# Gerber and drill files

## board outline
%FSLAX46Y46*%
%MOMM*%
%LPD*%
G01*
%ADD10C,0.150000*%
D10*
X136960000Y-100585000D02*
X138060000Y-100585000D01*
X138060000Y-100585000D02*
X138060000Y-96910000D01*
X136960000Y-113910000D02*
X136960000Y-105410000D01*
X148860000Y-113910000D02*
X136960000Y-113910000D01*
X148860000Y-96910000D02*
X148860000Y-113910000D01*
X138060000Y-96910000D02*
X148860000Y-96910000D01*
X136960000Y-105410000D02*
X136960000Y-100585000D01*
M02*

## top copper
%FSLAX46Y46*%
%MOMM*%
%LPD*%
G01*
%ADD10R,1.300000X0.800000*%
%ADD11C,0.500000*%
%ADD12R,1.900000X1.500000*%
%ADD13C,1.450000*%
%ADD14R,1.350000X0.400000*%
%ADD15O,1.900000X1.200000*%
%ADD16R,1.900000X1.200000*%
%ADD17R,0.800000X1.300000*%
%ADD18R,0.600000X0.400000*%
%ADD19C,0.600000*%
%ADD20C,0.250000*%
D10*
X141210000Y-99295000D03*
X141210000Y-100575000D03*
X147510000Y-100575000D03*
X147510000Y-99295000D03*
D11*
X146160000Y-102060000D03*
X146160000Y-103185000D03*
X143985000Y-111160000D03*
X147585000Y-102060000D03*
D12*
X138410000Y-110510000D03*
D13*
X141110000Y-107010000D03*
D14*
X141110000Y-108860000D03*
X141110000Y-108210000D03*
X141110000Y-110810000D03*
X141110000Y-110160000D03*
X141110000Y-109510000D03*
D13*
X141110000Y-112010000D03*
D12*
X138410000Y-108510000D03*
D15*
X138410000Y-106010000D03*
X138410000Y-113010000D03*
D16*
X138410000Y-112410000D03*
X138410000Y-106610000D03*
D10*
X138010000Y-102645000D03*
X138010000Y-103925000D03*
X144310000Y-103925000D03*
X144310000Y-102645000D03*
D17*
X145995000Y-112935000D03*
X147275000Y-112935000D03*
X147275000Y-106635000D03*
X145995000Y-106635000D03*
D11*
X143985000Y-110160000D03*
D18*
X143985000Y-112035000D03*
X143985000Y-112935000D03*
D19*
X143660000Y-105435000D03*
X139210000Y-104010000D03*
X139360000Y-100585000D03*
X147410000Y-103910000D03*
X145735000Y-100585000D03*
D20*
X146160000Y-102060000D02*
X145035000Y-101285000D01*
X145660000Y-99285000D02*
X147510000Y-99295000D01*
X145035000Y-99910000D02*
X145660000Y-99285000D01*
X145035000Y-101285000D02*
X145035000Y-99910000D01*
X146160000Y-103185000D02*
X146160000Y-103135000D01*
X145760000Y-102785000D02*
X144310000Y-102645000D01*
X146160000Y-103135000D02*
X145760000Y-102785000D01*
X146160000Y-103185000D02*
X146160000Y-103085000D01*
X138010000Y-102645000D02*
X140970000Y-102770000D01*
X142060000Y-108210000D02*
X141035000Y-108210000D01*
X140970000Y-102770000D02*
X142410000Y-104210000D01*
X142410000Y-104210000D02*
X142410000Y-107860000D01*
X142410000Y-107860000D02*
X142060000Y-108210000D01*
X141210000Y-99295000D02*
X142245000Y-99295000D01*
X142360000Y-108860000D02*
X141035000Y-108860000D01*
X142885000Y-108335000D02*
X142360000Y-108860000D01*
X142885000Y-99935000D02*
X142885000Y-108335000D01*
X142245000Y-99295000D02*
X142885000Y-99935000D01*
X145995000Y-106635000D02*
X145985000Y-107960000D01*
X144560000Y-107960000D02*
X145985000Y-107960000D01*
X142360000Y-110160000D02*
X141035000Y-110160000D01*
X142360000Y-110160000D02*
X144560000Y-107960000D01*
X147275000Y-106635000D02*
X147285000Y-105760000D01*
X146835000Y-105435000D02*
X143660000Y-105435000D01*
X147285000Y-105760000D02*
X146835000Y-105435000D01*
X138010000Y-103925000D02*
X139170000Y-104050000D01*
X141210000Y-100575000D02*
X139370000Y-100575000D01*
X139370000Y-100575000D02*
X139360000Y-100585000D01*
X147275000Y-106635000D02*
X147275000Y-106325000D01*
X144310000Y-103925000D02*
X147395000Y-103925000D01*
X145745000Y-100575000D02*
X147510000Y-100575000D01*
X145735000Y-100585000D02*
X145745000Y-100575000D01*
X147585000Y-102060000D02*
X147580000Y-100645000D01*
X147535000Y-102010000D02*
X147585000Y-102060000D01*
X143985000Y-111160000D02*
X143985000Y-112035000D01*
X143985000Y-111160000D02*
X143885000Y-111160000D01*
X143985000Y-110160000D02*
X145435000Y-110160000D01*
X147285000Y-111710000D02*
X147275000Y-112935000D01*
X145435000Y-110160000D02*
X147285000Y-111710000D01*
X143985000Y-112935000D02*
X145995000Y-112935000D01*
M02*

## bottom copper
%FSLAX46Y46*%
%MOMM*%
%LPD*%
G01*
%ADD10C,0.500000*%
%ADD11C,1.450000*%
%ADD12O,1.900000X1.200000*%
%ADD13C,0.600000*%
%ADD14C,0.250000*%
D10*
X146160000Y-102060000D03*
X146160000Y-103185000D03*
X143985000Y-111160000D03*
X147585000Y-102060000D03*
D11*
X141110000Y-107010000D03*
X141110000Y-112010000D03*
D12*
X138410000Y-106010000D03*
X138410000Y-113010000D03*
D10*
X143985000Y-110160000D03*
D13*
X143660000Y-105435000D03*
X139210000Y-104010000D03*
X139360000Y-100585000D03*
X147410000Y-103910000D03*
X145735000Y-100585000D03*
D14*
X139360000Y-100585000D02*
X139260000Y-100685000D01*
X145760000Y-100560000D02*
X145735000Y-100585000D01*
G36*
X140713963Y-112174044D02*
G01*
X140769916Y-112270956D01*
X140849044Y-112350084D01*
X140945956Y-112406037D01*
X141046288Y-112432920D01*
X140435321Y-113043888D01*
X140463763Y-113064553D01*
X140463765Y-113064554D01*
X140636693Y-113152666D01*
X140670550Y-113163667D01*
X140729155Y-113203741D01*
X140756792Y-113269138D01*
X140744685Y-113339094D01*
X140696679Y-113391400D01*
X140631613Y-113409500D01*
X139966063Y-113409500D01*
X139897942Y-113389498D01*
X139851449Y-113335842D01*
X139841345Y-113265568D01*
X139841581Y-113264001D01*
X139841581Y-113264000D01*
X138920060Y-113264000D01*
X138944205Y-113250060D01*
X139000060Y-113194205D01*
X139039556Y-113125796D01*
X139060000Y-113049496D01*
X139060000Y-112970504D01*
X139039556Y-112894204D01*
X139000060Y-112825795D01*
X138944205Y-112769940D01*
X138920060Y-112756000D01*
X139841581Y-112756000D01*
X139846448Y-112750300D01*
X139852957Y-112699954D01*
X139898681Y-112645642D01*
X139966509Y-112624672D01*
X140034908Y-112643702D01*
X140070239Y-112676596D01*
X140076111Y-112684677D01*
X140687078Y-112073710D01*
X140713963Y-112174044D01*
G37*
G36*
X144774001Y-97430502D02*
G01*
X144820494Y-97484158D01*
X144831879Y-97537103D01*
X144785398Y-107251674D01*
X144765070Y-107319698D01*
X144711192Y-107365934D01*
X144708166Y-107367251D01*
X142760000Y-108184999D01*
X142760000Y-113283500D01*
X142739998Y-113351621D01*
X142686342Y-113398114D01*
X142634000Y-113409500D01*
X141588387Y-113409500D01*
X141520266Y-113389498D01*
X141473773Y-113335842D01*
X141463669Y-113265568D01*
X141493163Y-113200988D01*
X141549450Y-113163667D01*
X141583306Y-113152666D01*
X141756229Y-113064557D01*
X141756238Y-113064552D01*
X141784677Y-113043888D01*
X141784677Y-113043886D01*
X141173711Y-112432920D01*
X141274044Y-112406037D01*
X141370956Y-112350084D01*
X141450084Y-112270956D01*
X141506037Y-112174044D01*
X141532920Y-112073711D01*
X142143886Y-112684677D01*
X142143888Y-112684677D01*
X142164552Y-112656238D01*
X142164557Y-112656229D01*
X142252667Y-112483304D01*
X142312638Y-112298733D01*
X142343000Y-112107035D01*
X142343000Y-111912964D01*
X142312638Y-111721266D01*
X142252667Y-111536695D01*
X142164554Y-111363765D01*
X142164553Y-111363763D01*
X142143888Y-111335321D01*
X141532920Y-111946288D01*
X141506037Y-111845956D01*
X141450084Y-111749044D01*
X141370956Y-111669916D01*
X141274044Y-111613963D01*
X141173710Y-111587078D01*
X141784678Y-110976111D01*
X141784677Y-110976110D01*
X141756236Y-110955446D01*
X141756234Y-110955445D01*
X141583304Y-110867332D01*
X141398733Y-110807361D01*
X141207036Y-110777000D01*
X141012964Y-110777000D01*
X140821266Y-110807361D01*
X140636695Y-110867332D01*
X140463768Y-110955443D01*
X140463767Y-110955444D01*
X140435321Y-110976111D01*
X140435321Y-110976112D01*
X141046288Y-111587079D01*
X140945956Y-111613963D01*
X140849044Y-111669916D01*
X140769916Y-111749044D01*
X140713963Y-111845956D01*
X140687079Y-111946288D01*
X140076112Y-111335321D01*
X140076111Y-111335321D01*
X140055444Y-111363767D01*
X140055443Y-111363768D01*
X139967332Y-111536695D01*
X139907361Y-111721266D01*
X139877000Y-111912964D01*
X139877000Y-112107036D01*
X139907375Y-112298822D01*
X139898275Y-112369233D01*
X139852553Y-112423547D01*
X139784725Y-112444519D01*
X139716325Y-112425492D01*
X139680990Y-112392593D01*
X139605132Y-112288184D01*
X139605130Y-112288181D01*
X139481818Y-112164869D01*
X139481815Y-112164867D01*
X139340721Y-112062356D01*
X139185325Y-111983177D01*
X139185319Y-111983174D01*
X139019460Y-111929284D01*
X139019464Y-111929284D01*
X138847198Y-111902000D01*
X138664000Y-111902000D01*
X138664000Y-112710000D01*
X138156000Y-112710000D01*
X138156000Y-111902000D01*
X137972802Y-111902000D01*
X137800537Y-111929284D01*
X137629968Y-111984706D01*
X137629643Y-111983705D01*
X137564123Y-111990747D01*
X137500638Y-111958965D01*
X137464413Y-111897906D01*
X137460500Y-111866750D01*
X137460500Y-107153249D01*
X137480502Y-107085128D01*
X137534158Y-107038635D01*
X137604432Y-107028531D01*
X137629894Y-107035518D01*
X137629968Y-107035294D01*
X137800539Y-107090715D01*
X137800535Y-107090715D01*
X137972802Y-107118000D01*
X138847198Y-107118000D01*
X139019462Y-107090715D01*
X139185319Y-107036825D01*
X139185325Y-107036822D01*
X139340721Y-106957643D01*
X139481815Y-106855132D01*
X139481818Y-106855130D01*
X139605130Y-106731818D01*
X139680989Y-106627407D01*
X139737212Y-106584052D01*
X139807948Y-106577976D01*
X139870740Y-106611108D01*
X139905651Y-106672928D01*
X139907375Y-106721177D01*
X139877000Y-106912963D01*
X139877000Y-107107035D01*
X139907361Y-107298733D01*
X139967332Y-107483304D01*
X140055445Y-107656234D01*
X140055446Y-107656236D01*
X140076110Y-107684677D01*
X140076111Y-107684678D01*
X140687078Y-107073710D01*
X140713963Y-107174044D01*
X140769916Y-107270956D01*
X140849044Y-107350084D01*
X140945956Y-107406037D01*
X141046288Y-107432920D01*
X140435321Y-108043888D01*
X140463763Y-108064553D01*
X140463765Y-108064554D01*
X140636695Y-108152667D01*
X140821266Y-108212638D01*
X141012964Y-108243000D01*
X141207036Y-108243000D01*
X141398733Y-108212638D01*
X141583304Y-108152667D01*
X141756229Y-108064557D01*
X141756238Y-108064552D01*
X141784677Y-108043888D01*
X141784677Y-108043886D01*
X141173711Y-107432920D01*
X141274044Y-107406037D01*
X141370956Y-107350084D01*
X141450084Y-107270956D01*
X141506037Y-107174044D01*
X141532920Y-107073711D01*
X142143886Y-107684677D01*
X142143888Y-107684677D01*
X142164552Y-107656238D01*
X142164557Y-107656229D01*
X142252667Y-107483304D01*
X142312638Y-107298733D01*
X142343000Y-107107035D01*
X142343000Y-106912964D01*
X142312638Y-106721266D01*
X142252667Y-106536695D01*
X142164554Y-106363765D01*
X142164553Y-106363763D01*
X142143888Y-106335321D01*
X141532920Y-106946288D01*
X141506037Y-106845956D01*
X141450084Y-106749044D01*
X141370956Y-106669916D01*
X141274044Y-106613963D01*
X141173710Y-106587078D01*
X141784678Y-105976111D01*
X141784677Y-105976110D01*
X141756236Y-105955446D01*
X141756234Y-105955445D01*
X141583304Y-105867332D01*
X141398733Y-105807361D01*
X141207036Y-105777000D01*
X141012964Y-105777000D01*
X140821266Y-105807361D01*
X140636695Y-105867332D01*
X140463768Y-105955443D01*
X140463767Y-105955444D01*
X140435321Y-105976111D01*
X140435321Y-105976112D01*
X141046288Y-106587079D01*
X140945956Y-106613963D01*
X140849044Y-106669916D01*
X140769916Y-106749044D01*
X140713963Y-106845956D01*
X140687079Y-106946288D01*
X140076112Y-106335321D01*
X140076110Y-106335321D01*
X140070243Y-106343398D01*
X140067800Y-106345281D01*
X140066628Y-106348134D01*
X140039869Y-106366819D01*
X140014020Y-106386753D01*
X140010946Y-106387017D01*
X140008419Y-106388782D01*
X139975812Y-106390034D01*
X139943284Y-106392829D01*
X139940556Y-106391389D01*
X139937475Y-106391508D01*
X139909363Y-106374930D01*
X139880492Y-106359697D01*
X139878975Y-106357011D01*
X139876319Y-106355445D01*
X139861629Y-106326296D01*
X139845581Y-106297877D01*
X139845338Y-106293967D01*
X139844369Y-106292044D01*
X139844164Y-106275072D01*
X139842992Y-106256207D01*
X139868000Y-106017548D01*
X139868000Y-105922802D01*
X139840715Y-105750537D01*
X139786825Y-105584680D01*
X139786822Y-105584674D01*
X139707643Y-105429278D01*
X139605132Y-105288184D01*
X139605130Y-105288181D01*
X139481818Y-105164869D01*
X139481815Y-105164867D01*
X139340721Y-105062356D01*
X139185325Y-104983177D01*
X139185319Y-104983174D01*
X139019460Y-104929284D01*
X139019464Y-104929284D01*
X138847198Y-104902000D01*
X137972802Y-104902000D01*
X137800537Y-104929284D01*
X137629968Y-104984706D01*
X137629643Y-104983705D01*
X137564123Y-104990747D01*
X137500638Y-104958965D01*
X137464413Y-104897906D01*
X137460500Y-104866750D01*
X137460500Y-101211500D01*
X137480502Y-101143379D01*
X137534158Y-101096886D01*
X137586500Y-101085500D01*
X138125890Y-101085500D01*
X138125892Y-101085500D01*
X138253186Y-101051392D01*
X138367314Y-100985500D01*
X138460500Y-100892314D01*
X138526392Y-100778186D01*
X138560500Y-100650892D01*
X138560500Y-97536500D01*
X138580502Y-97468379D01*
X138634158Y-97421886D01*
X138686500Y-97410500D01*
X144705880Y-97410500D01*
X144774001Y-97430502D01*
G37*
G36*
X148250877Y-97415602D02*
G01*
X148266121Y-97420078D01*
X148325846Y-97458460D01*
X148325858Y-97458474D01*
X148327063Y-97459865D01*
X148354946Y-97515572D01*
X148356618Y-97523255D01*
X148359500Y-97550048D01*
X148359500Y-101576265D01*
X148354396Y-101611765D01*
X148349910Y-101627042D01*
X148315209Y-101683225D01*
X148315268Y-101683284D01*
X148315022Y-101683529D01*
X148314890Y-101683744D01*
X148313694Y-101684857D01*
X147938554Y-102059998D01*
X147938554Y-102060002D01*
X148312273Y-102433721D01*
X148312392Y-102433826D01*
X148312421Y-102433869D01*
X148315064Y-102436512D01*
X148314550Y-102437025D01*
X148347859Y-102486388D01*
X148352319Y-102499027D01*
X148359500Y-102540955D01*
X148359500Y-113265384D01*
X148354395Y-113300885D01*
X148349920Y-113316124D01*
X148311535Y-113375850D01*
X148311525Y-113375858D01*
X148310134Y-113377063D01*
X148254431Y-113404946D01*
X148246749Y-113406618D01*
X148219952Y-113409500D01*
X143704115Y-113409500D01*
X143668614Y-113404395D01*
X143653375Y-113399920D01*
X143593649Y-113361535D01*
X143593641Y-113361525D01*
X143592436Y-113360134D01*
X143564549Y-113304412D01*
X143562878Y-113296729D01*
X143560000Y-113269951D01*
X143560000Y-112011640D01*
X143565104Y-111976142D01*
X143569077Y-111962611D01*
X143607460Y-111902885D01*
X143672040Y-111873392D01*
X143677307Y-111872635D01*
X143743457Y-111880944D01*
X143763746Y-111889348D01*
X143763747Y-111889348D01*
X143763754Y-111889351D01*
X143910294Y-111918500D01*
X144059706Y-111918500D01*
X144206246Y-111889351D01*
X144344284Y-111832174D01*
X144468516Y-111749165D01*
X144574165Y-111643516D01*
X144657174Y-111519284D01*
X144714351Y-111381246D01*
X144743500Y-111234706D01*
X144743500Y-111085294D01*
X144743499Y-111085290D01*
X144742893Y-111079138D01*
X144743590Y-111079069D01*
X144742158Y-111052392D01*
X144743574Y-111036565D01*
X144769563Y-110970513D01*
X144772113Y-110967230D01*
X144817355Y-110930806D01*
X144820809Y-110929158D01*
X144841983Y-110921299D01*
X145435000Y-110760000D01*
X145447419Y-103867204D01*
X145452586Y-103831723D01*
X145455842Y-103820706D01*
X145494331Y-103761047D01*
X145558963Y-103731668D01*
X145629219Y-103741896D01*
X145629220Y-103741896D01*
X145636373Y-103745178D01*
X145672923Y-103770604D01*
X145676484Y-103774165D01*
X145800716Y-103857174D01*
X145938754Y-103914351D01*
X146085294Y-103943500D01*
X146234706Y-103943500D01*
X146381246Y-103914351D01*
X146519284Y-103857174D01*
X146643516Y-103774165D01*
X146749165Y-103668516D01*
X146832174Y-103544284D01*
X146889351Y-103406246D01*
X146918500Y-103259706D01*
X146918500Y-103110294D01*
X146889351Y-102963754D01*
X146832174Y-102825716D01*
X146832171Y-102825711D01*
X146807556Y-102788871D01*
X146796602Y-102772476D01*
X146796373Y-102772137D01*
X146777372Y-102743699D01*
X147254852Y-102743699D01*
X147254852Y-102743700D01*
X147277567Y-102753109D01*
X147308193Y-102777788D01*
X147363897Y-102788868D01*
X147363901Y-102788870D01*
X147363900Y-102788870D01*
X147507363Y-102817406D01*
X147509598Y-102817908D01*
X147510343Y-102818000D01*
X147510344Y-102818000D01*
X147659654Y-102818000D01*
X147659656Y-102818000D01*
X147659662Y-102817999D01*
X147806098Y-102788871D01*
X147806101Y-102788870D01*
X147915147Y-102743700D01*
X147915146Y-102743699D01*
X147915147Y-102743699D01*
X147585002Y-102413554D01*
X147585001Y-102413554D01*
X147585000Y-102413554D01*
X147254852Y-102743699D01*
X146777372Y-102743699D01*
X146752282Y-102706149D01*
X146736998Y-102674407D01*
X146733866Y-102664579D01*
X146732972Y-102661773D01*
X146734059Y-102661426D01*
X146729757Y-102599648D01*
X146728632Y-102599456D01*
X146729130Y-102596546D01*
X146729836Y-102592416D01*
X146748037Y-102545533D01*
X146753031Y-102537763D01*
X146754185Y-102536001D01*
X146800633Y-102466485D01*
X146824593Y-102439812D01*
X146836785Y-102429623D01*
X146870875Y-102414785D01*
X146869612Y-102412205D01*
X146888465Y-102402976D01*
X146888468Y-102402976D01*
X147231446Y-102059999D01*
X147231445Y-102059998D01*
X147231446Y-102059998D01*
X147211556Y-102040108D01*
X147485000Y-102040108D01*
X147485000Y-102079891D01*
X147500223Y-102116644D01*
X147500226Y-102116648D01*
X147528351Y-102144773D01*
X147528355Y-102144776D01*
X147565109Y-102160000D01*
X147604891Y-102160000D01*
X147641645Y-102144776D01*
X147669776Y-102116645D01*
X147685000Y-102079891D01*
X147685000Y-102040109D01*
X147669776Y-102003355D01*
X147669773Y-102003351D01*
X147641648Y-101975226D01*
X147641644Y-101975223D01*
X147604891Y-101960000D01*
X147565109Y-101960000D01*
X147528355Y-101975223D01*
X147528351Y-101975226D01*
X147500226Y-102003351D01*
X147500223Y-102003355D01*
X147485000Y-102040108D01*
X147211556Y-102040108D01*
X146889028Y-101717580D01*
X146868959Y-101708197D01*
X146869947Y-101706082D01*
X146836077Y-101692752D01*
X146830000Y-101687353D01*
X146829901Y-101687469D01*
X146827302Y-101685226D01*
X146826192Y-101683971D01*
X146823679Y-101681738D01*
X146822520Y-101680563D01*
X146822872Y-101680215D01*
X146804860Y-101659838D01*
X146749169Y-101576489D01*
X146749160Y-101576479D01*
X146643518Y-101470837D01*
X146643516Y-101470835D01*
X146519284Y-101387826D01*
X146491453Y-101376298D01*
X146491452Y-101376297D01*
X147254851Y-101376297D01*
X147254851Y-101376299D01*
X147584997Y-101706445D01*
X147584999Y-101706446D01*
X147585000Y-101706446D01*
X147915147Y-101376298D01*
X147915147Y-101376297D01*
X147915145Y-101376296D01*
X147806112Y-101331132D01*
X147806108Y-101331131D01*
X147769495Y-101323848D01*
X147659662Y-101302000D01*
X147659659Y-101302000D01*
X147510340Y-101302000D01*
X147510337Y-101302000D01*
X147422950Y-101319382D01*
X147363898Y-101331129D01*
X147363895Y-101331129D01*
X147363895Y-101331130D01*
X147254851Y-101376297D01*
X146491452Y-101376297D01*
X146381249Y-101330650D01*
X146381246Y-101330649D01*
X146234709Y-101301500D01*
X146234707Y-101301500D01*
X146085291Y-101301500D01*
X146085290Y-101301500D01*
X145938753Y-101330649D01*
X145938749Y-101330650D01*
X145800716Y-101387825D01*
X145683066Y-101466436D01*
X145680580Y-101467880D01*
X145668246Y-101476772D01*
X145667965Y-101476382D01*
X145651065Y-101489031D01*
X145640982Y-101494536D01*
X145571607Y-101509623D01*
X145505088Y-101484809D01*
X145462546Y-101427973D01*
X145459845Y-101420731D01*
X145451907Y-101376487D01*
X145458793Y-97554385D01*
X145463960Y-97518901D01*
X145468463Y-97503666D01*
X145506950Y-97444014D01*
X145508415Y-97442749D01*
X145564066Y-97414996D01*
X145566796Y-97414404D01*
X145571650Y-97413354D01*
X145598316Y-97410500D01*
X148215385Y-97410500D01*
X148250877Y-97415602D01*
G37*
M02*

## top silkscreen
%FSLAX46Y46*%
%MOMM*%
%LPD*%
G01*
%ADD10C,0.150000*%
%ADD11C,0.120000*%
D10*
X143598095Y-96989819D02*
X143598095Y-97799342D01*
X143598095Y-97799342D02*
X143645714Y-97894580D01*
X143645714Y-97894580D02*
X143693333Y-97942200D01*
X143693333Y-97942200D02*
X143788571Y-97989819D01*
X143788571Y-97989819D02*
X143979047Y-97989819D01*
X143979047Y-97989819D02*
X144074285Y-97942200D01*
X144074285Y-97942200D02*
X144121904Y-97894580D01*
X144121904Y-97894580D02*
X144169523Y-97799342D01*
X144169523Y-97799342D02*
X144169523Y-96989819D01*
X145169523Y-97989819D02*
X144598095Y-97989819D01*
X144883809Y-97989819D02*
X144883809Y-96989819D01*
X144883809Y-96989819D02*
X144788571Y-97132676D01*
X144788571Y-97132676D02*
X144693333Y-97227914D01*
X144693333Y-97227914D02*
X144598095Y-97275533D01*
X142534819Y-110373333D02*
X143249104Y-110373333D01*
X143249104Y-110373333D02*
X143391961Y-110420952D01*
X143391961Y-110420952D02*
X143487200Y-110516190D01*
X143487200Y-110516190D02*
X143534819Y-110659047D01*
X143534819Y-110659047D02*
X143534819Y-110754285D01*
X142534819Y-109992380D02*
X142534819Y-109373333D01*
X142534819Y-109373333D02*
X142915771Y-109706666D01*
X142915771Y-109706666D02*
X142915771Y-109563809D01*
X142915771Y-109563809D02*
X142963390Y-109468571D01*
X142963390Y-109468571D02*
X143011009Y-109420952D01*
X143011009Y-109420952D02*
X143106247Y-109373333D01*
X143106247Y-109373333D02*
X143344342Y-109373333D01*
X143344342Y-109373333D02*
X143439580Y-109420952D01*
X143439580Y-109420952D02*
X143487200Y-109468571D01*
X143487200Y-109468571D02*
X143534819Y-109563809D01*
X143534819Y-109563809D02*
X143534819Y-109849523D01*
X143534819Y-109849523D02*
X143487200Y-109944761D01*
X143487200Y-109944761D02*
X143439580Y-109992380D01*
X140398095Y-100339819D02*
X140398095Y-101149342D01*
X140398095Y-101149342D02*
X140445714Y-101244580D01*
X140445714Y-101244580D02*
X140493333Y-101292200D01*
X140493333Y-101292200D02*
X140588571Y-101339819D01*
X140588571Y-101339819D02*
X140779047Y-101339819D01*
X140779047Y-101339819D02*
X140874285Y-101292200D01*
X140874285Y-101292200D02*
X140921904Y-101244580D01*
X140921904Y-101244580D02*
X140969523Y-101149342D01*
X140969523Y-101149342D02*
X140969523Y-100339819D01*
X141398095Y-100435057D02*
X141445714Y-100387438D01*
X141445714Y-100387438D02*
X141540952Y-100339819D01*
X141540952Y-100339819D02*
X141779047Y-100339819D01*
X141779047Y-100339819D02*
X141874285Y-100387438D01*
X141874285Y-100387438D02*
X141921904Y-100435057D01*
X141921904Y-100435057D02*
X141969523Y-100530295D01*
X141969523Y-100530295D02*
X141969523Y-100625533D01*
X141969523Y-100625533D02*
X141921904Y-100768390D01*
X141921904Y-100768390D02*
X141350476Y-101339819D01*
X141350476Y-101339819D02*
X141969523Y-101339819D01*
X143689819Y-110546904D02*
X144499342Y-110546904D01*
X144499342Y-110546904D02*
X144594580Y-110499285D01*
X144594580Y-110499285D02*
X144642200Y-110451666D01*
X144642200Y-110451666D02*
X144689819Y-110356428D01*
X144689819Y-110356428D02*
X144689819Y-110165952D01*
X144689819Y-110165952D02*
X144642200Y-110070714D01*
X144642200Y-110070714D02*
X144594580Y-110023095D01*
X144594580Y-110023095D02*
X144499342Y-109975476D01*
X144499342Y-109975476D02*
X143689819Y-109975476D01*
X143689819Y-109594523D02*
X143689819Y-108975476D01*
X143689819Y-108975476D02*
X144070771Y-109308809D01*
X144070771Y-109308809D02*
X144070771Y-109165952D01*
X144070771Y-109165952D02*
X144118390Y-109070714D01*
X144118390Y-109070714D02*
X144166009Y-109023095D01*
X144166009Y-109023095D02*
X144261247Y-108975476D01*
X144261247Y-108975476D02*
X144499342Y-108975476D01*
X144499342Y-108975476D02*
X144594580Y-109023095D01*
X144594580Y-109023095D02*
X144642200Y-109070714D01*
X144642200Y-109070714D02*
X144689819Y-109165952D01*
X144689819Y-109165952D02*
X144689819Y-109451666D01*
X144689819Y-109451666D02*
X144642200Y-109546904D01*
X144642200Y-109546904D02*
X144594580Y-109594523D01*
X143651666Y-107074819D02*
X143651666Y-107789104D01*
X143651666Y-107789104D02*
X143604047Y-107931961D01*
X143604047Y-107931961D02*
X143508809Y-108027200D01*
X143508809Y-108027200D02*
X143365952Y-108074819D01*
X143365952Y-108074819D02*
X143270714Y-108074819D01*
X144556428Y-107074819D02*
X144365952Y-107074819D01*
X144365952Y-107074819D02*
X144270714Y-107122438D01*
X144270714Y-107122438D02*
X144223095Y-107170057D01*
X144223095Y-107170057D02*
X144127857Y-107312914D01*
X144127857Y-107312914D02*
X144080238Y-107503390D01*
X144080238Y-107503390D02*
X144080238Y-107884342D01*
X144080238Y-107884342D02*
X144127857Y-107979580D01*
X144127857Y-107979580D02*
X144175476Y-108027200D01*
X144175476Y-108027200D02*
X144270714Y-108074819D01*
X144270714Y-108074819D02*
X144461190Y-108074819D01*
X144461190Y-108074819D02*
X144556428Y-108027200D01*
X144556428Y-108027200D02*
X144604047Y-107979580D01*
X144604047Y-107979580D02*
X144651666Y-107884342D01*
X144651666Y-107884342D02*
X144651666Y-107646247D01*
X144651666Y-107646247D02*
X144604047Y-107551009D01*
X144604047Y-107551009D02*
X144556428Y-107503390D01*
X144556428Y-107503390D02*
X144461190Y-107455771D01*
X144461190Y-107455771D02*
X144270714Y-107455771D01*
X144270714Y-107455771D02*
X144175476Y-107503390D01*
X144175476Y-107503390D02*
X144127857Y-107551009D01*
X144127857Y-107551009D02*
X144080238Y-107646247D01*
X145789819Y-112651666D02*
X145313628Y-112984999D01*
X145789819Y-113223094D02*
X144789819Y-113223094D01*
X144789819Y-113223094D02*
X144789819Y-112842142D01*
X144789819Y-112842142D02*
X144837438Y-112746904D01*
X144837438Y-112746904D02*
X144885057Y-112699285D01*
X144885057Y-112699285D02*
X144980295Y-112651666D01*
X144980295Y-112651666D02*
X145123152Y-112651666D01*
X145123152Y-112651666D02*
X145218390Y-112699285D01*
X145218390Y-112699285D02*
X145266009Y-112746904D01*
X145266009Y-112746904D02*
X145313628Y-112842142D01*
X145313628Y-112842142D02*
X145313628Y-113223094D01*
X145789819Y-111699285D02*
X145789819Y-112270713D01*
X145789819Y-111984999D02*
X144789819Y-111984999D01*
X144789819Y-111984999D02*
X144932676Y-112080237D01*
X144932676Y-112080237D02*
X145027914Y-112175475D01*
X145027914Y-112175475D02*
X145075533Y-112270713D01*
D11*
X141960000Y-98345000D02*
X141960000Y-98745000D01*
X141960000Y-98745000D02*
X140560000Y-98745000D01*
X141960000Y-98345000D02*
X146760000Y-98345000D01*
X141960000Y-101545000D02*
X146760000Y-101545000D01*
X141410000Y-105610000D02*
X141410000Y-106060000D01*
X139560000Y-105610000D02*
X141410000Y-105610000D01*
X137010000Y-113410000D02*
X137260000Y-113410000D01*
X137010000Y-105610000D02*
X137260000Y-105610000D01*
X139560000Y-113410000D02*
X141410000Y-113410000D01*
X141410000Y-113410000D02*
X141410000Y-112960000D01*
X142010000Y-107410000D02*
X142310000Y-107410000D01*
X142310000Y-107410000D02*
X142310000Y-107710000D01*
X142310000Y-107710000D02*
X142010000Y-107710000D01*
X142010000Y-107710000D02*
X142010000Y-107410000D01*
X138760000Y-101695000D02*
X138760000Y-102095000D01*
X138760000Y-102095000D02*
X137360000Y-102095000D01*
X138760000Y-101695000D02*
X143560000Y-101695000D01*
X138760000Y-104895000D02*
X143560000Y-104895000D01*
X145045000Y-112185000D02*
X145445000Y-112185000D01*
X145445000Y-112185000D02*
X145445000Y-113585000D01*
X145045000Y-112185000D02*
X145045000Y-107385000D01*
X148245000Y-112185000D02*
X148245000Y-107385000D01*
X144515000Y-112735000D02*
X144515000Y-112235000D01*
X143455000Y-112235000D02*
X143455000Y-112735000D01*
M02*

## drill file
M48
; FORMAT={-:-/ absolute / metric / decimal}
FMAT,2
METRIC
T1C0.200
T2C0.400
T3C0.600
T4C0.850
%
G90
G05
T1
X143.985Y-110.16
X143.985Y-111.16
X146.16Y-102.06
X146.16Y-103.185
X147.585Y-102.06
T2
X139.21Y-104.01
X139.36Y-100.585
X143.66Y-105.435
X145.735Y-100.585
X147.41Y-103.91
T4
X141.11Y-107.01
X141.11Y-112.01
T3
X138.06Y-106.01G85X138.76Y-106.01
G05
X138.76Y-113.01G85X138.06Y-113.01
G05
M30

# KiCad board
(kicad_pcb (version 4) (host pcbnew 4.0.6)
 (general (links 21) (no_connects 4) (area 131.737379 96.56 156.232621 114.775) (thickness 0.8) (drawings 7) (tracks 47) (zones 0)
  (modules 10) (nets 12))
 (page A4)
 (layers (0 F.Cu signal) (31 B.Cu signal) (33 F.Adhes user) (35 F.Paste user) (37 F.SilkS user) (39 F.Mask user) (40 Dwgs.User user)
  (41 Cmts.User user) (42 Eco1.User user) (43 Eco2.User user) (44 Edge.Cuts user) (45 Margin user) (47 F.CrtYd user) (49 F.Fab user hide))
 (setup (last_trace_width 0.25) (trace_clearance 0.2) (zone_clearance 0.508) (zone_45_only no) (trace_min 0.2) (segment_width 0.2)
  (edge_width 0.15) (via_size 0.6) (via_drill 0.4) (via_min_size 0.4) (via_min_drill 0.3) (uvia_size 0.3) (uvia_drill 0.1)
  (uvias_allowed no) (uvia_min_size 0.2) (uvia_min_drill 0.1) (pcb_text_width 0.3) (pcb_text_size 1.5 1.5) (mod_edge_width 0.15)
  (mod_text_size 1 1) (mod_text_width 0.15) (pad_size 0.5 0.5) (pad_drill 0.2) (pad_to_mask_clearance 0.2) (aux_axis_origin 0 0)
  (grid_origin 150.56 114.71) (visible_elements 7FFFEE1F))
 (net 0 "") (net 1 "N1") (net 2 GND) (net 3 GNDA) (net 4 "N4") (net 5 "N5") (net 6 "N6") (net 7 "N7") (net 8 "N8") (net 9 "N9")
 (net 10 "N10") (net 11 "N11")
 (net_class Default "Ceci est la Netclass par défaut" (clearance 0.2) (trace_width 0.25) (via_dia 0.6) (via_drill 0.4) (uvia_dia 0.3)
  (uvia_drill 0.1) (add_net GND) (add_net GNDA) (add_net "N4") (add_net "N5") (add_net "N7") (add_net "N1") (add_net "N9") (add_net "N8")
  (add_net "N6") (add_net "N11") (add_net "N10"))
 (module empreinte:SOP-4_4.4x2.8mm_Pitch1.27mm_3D (layer F.Cu) (at 144.36 99.935)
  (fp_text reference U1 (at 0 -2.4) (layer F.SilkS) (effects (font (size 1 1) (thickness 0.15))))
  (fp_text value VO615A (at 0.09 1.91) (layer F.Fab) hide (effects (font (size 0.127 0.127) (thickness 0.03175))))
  (fp_line (start -2.4 -1.59) (end -2.4 -1.19) (layer F.SilkS) (width 0.12))
  (fp_line (start -2.4 -1.19) (end -3.8 -1.19) (layer F.SilkS) (width 0.12))
  (fp_line (start -2.4 -1.59) (end 2.4 -1.59) (layer F.SilkS) (width 0.12))
  (fp_line (start -2.4 1.61) (end 2.4 1.61) (layer F.SilkS) (width 0.12))
  (pad 1 smd rect (at -3.15 -0.64) (size 1.3 0.8) (layers F.Cu F.Paste F.Mask) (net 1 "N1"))
  (pad 2 smd rect (at -3.15 0.64) (size 1.3 0.8) (layers F.Cu F.Paste F.Mask) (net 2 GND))
  (pad 3 smd rect (at 3.15 0.64) (size 1.3 0.8) (layers F.Cu F.Paste F.Mask) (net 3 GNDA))
  (pad 4 smd rect (at 3.15 -0.64) (size 1.3 0.8) (layers F.Cu F.Paste F.Mask) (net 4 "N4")))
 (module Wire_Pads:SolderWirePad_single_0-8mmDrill (layer F.Cu) (at 146.16 102.06)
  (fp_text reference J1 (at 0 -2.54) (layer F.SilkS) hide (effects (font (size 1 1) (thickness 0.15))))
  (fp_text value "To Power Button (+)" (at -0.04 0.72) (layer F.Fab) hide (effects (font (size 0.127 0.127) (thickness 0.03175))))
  (pad 1 thru_hole circle (at 0 0) (size 0.5 0.5) (drill 0.2) (layers *.Cu *.Mask) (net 4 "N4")))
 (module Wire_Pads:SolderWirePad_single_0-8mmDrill (layer F.Cu) (at 146.16 103.185)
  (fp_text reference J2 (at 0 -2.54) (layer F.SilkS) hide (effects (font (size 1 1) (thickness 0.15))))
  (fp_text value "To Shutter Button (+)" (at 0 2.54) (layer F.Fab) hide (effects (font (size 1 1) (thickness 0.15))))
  (pad 1 thru_hole circle (at 0 0) (size 0.5 0.5) (drill 0.2) (layers *.Cu *.Mask) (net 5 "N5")))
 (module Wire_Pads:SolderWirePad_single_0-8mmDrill (layer F.Cu) (at 143.985 111.16)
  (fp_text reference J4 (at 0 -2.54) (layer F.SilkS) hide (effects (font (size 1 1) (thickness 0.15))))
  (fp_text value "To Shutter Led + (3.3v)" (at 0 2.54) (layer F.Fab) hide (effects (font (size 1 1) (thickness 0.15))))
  (pad 1 thru_hole circle (at 0 0) (size 0.5 0.5) (drill 0.2) (layers *.Cu *.Mask) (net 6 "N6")))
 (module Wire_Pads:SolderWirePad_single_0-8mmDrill (layer F.Cu) (at 147.585 102.06)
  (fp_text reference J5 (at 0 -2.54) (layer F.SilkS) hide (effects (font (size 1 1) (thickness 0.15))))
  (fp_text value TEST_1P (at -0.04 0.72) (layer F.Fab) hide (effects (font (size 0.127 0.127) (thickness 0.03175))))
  (pad 1 thru_hole circle (at 0 0) (size 0.5 0.5) (drill 0.2) (layers *.Cu *.Mask) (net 3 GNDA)))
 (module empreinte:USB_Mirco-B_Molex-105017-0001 (layer F.Cu) (at 141.11 109.51 270)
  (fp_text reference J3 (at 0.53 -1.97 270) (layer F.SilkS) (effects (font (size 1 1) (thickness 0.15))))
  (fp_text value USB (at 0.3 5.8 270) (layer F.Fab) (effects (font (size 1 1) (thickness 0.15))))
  (fp_line (start -3.9 -0.3) (end -3.45 -0.3) (layer F.SilkS) (width 0.12))
  (fp_line (start -3.9 1.55) (end -3.9 -0.3) (layer F.SilkS) (width 0.12))
  (fp_line (start 3.9 4.1) (end 3.9 3.85) (layer F.SilkS) (width 0.12))
  (fp_line (start -3.9 4.1) (end -3.9 3.85) (layer F.SilkS) (width 0.12))
  (fp_line (start 3.9 1.55) (end 3.9 -0.3) (layer F.SilkS) (width 0.12))
  (fp_line (start 3.9 -0.3) (end 3.45 -0.3) (layer F.SilkS) (width 0.12))
  (fp_line (start -2.1 -0.9) (end -2.1 -1.2) (layer F.SilkS) (width 0.12))
  (fp_line (start -2.1 -1.2) (end -1.8 -1.2) (layer F.SilkS) (width 0.12))
  (fp_line (start -1.8 -1.2) (end -1.8 -0.9) (layer F.SilkS) (width 0.12))
  (fp_line (start -1.8 -0.9) (end -2.1 -0.9) (layer F.SilkS) (width 0.12))
  (pad 6 smd rect (at 1 2.7 270) (size 1.5 1.9) (layers F.Cu F.Paste F.Mask) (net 2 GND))
  (pad 6 thru_hole circle (at -2.5 0 270) (size 1.45 1.45) (drill 0.85) (layers *.Cu *.Mask) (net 2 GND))
  (pad 2 smd rect (at -0.65 0 270) (size 0.4 1.35) (layers F.Cu F.Paste F.Mask) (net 1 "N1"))
  (pad 1 smd rect (at -1.3 0 270) (size 0.4 1.35) (layers F.Cu F.Paste F.Mask) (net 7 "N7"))
  (pad 5 smd rect (at 1.3 0 270) (size 0.4 1.35) (layers F.Cu F.Paste F.Mask) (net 2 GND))
  (pad 4 smd rect (at 0.65 0 270) (size 0.4 1.35) (layers F.Cu F.Paste F.Mask) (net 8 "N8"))
  (pad 3 smd rect (at 0 0 270) (size 0.4 1.35) (layers F.Cu F.Paste F.Mask) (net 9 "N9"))
  (pad 6 thru_hole circle (at 2.5 0 270) (size 1.45 1.45) (drill 0.85) (layers *.Cu *.Mask) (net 2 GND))
  (pad 6 smd rect (at -1 2.7 270) (size 1.5 1.9) (layers F.Cu F.Paste F.Mask) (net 2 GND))
  (pad 6 thru_hole oval (at -3.5 2.7 90) (size 1.2 1.9) (drill oval 0.6 1.3) (layers *.Cu *.Mask) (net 2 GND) (zone_connect 0))
  (pad 6 thru_hole oval (at 3.5 2.7 270) (size 1.2 1.9) (drill oval 0.6 1.3) (layers *.Cu *.Mask) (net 2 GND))
  (pad 6 smd rect (at 2.9 2.7 270) (size 1.2 1.9) (layers F.Cu F.Mask) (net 2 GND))
  (pad 6 smd rect (at -2.9 2.7 270) (size 1.2 1.9) (layers F.Cu F.Mask) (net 2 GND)))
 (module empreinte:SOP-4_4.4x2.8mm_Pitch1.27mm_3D (layer F.Cu) (at 141.16 103.285)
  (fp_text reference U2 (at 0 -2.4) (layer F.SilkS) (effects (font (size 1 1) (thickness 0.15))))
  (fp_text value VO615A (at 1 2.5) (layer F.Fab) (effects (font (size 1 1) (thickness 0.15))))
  (fp_line (start -2.4 -1.59) (end -2.4 -1.19) (layer F.SilkS) (width 0.12))
  (fp_line (start -2.4 -1.19) (end -3.8 -1.19) (layer F.SilkS) (width 0.12))
  (fp_line (start -2.4 -1.59) (end 2.4 -1.59) (layer F.SilkS) (width 0.12))
  (fp_line (start -2.4 1.61) (end 2.4 1.61) (layer F.SilkS) (width 0.12))
  (pad 1 smd rect (at -3.15 -0.64) (size 1.3 0.8) (layers F.Cu F.Paste F.Mask) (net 7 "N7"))
  (pad 2 smd rect (at -3.15 0.64) (size 1.3 0.8) (layers F.Cu F.Paste F.Mask) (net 2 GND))
  (pad 3 smd rect (at 3.15 0.64) (size 1.3 0.8) (layers F.Cu F.Paste F.Mask) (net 3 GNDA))
  (pad 4 smd rect (at 3.15 -0.64) (size 1.3 0.8) (layers F.Cu F.Paste F.Mask) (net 5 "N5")))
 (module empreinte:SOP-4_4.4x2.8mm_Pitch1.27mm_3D (layer F.Cu) (at 146.635 109.785 90)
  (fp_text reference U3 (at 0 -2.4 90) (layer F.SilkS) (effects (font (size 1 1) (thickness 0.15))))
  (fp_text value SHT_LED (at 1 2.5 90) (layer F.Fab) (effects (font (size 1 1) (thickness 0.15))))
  (fp_line (start -2.4 -1.59) (end -2.4 -1.19) (layer F.SilkS) (width 0.12))
  (fp_line (start -2.4 -1.19) (end -3.8 -1.19) (layer F.SilkS) (width 0.12))
  (fp_line (start -2.4 -1.59) (end 2.4 -1.59) (layer F.SilkS) (width 0.12))
  (fp_line (start -2.4 1.61) (end 2.4 1.61) (layer F.SilkS) (width 0.12))
  (pad 1 smd rect (at -3.15 -0.64 90) (size 1.3 0.8) (layers F.Cu F.Paste F.Mask) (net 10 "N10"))
  (pad 2 smd rect (at -3.15 0.64 90) (size 1.3 0.8) (layers F.Cu F.Paste F.Mask) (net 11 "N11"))
  (pad 3 smd rect (at 3.15 0.64 90) (size 1.3 0.8) (layers F.Cu F.Paste F.Mask) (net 2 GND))
  (pad 4 smd rect (at 3.15 -0.64 90) (size 1.3 0.8) (layers F.Cu F.Paste F.Mask) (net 8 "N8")))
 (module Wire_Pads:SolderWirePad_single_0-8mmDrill (layer F.Cu) (at 143.985 110.16)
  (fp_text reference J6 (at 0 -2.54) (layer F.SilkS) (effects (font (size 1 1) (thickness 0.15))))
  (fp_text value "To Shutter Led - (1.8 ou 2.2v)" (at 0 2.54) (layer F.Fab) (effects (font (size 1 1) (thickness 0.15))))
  (pad 1 thru_hole circle (at 0 0) (size 0.5 0.5) (drill 0.2) (layers *.Cu *.Mask) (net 11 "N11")))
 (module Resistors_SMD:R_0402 (layer F.Cu) (at 143.985 112.485 270)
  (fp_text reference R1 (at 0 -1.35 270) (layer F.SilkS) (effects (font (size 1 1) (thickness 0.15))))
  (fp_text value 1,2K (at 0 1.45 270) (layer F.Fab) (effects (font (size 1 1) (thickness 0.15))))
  (fp_line (start 0.25 -0.53) (end -0.25 -0.53) (layer F.SilkS) (width 0.12))
  (fp_line (start -0.25 0.53) (end 0.25 0.53) (layer F.SilkS) (width 0.12))
  (pad 1 smd rect (at -0.45 0 270) (size 0.4 0.6) (layers F.Cu F.Paste F.Mask) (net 6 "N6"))
  (pad 2 smd rect (at 0.45 0 270) (size 0.4 0.6) (layers F.Cu F.Paste F.Mask) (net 10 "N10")))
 (gr_line (start 136.96 100.585) (end 138.06 100.585) (layer Edge.Cuts) (width 0.15))
 (gr_line (start 138.06 100.585) (end 138.06 96.91) (angle 90) (layer Edge.Cuts) (width 0.15))
 (gr_line (start 136.96 113.91) (end 136.96 105.41) (angle 90) (layer Edge.Cuts) (width 0.15))
 (gr_line (start 148.86 113.91) (end 136.96 113.91) (angle 90) (layer Edge.Cuts) (width 0.15))
 (gr_line (start 148.86 96.91) (end 148.86 113.91) (angle 90) (layer Edge.Cuts) (width 0.15))
 (gr_line (start 138.06 96.91) (end 148.86 96.91) (angle 90) (layer Edge.Cuts) (width 0.15))
 (gr_line (start 136.96 105.41) (end 136.96 100.585) (angle 90) (layer Edge.Cuts) (width 0.15))
 (segment (start 146.16 102.06) (end 145.035 101.285) (width 0.25) (layer F.Cu) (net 4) (status 10))
 (segment (start 145.66 99.285) (end 147.51 99.295) (width 0.25) (layer F.Cu) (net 4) (status 20))
 (segment (start 145.035 99.91) (end 145.66 99.285) (width 0.25) (layer F.Cu) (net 4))
 (segment (start 145.035 101.285) (end 145.035 99.91) (width 0.25) (layer F.Cu) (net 4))
 (segment (start 146.16 103.185) (end 146.16 103.135) (width 0.25) (layer F.Cu) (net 5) (status 30))
 (segment (start 145.76 102.785) (end 144.31 102.645) (width 0.25) (layer F.Cu) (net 5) (status 20))
 (segment (start 146.16 103.135) (end 145.76 102.785) (width 0.25) (layer F.Cu) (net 5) (status 10))
 (segment (start 146.16 103.185) (end 146.16 103.085) (width 0.25) (layer F.Cu) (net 5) (status 30))
 (segment (start 138.01 102.645) (end 140.97 102.77) (width 0.25) (layer F.Cu) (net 7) (status 10))
 (segment (start 142.06 108.21) (end 141.035 108.21) (width 0.25) (layer F.Cu) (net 7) (status 20))
 (segment (start 140.97 102.77) (end 142.41 104.21) (width 0.25) (layer F.Cu) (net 7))
 (segment (start 142.41 104.21) (end 142.41 107.86) (width 0.25) (layer F.Cu) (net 7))
 (segment (start 142.41 107.86) (end 142.06 108.21) (width 0.25) (layer F.Cu) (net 7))
 (segment (start 141.21 99.295) (end 142.245 99.295) (width 0.25) (layer F.Cu) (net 1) (status 10))
 (segment (start 142.36 108.86) (end 141.035 108.86) (width 0.25) (layer F.Cu) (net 1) (status 20))
 (segment (start 142.885 108.335) (end 142.36 108.86) (width 0.25) (layer F.Cu) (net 1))
 (segment (start 142.885 99.935) (end 142.885 108.335) (width 0.25) (layer F.Cu) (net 1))
 (segment (start 142.245 99.295) (end 142.885 99.935) (width 0.25) (layer F.Cu) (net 1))
 (segment (start 145.995 106.635) (end 145.985 107.96) (width 0.25) (layer F.Cu) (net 8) (status 10))
 (segment (start 144.56 107.96) (end 145.985 107.96) (width 0.25) (layer F.Cu) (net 8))
 (segment (start 142.36 110.16) (end 141.035 110.16) (width 0.25) (layer F.Cu) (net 8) (status 20))
 (segment (start 142.36 110.16) (end 144.56 107.96) (width 0.25) (layer F.Cu) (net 8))
 (segment (start 147.275 106.635) (end 147.285 105.76) (width 0.25) (layer F.Cu) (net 2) (status 10))
 (via (at 143.66 105.435) (size 0.6) (drill 0.4) (layers F.Cu B.Cu) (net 2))
 (segment (start 146.835 105.435) (end 143.66 105.435) (width 0.25) (layer F.Cu) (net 2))
 (segment (start 147.285 105.76) (end 146.835 105.435) (width 0.25) (layer F.Cu) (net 2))
 (segment (start 138.01 103.925) (end 139.17 104.05) (width 0.25) (layer F.Cu) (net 2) (status 10))
 (via (at 139.21 104.01) (size 0.6) (drill 0.4) (layers F.Cu B.Cu) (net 2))
 (segment (start 141.21 100.575) (end 139.37 100.575) (width 0.25) (layer F.Cu) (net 2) (status 10))
 (via (at 139.36 100.585) (size 0.6) (drill 0.4) (layers F.Cu B.Cu) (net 2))
 (segment (start 139.36 100.585) (end 139.26 100.685) (width 0.25) (layer B.Cu) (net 2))
 (segment (start 139.37 100.575) (end 139.36 100.585) (width 0.25) (layer F.Cu) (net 2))
 (segment (start 147.275 106.635) (end 147.275 106.325) (width 0.25) (layer F.Cu) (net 2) (status 30))
 (segment (start 144.31 103.925) (end 147.395 103.925) (width 0.25) (layer F.Cu) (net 3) (status 10))
 (via (at 147.41 103.91) (size 0.6) (drill 0.4) (layers F.Cu B.Cu) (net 3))
 (segment (start 145.76 100.56) (end 145.735 100.585) (width 0.25) (layer B.Cu) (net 3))
 (segment (start 145.745 100.575) (end 147.51 100.575) (width 0.25) (layer F.Cu) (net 3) (status 20))
 (segment (start 145.735 100.585) (end 145.745 100.575) (width 0.25) (layer F.Cu) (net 3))
 (via (at 145.735 100.585) (size 0.6) (drill 0.4) (layers F.Cu B.Cu) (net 3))
 (segment (start 147.585 102.06) (end 147.58 100.645) (width 0.25) (layer F.Cu) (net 3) (status 10))
 (segment (start 147.535 102.01) (end 147.585 102.06) (width 0.25) (layer F.Cu) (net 3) (status 30))
 (segment (start 143.985 111.16) (end 143.985 112.035) (width 0.25) (layer F.Cu) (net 6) (status 10))
 (segment (start 143.985 111.16) (end 143.885 111.16) (width 0.25) (layer F.Cu) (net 6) (status 30))
 (segment (start 143.985 110.16) (end 145.435 110.16) (width 0.25) (layer F.Cu) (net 11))
 (segment (start 147.285 111.71) (end 147.275 112.935) (width 0.25) (layer F.Cu) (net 11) (status 20))
 (segment (start 145.435 110.16) (end 147.285 111.71) (width 0.25) (layer F.Cu) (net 11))
 (segment (start 143.985 112.935) (end 145.995 112.935) (width 0.25) (layer F.Cu) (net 10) (status 20))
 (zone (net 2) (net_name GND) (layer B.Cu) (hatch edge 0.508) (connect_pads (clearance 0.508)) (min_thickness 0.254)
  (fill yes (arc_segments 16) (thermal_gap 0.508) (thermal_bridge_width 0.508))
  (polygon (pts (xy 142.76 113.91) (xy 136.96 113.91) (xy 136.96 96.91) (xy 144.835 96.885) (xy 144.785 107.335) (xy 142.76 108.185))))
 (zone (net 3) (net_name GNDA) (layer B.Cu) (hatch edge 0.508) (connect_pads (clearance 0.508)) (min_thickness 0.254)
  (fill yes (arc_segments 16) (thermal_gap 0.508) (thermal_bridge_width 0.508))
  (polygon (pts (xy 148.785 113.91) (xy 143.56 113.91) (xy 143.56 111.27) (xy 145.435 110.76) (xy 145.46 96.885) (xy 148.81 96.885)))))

